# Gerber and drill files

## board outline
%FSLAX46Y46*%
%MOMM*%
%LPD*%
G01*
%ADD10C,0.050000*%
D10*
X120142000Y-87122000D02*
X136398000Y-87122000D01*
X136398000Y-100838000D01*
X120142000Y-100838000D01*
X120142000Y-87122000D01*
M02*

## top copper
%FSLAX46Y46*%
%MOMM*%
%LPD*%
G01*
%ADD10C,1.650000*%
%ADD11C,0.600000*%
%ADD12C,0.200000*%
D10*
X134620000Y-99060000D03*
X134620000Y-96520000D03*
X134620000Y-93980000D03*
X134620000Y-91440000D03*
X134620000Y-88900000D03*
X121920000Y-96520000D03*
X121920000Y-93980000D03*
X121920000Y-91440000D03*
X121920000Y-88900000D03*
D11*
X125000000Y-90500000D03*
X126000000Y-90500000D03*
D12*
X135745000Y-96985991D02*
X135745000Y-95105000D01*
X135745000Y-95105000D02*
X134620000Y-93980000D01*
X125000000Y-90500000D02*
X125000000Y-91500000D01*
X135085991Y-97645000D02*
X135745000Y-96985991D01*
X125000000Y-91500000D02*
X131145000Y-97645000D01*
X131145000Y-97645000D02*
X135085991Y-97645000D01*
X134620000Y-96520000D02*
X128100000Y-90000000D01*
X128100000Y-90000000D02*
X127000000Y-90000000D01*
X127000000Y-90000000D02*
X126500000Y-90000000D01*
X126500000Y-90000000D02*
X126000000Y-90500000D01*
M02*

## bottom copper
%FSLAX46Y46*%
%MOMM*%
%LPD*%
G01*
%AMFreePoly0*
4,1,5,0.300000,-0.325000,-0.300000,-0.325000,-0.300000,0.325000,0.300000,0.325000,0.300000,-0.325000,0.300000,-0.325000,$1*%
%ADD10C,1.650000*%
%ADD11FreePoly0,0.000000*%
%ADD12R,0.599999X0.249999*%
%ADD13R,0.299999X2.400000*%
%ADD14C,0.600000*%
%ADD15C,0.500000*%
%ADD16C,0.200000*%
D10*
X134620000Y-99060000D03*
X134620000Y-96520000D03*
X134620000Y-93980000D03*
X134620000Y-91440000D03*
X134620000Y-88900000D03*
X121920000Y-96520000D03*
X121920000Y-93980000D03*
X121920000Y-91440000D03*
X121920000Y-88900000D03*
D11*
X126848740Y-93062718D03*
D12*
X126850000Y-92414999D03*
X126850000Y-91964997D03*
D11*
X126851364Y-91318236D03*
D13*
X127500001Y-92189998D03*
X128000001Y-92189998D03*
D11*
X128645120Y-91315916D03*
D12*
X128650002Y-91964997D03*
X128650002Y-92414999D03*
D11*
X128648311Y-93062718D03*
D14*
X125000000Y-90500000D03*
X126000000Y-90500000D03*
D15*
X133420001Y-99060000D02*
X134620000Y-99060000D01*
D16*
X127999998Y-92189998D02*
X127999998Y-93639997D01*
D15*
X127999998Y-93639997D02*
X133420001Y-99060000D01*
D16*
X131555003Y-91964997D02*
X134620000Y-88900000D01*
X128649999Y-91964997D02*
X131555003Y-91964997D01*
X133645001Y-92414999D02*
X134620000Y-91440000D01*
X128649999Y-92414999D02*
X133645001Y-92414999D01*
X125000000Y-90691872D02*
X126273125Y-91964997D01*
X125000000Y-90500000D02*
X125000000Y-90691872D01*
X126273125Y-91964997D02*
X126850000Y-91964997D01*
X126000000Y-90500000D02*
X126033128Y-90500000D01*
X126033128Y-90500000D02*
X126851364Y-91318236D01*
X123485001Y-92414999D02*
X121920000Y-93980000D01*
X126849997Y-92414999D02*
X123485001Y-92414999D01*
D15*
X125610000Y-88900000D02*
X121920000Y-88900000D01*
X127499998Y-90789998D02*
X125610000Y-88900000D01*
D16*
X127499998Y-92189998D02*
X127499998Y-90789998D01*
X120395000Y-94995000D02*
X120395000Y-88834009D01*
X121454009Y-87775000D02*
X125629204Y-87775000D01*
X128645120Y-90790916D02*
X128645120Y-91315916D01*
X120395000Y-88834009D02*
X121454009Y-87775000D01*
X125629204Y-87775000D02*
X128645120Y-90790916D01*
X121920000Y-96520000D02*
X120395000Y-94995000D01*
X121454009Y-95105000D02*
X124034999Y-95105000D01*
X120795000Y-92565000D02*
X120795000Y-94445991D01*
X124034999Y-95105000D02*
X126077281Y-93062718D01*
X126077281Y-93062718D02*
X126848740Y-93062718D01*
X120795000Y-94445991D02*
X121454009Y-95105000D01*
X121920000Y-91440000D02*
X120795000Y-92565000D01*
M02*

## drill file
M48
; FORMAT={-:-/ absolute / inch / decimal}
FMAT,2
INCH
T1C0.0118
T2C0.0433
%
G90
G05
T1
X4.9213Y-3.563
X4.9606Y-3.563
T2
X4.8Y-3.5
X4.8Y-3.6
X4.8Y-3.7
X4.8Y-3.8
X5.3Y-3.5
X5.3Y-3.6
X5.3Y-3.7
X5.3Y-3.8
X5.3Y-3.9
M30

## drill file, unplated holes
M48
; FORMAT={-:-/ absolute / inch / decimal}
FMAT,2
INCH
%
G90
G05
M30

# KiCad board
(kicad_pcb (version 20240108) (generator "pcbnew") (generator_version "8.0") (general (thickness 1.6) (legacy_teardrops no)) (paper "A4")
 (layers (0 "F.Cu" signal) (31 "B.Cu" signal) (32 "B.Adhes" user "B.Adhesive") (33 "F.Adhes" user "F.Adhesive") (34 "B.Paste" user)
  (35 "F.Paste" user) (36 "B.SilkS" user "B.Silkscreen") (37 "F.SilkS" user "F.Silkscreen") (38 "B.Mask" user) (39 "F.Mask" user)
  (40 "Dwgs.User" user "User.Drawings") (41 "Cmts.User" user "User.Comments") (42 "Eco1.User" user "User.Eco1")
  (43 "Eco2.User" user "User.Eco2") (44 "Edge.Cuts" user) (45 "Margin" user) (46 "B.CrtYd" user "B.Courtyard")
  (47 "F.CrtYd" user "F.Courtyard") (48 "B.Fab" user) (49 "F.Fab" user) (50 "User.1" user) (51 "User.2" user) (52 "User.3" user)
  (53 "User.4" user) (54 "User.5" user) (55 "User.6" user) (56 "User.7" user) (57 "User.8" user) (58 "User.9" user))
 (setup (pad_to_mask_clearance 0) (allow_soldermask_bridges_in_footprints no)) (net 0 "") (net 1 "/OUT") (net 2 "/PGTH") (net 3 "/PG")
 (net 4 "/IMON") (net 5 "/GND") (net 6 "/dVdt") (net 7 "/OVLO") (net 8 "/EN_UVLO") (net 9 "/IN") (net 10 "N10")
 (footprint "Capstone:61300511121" (layer "F.Cu") (at 134.62 93.98 90)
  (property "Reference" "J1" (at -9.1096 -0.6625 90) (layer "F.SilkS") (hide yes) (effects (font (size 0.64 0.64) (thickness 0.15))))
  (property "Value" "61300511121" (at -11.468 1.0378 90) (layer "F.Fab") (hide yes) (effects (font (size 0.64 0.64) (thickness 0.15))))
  (pad "1" thru_hole circle (at -5.08 0 90) (size 1.65 1.65) (drill 1.1) (layers "*.Cu" "*.Mask") (remove_unused_layers no) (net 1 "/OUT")
   (solder_mask_margin 0.102))
  (pad "2" thru_hole circle (at -2.54 0 90) (size 1.65 1.65) (drill 1.1) (layers "*.Cu" "*.Mask") (remove_unused_layers no) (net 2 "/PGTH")
   (solder_mask_margin 0.102))
  (pad "3" thru_hole circle (at 0 0 90) (size 1.65 1.65) (drill 1.1) (layers "*.Cu" "*.Mask") (remove_unused_layers no) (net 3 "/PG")
   (solder_mask_margin 0.102))
  (pad "4" thru_hole circle (at 2.54 0 90) (size 1.65 1.65) (drill 1.1) (layers "*.Cu" "*.Mask") (remove_unused_layers no) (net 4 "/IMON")
   (solder_mask_margin 0.102))
  (pad "5" thru_hole circle (at 5.08 0 90) (size 1.65 1.65) (drill 1.1) (layers "*.Cu" "*.Mask") (remove_unused_layers no) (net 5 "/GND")
   (solder_mask_margin 0.102)))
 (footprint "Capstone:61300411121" (layer "F.Cu") (at 121.92 92.71 90)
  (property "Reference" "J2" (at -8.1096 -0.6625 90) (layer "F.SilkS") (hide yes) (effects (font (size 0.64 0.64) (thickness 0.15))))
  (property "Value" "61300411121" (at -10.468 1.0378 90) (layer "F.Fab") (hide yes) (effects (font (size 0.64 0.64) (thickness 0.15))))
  (pad "1" thru_hole circle (at -3.81 0 90) (size 1.65 1.65) (drill 1.1) (layers "*.Cu" "*.Mask") (remove_unused_layers no) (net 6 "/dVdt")
   (solder_mask_margin 0.102))
  (pad "2" thru_hole circle (at -1.27 0 90) (size 1.65 1.65) (drill 1.1) (layers "*.Cu" "*.Mask") (remove_unused_layers no) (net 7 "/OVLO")
   (solder_mask_margin 0.102))
  (pad "3" thru_hole circle (at 1.27 0 90) (size 1.65 1.65) (drill 1.1) (layers "*.Cu" "*.Mask") (remove_unused_layers no)
   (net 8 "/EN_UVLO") (solder_mask_margin 0.102))
  (pad "4" thru_hole circle (at 3.81 0 90) (size 1.65 1.65) (drill 1.1) (layers "*.Cu" "*.Mask") (remove_unused_layers no) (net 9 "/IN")
   (solder_mask_margin 0.102)))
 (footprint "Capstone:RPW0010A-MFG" (layer "B.Cu") (at 127.750001 92.189998)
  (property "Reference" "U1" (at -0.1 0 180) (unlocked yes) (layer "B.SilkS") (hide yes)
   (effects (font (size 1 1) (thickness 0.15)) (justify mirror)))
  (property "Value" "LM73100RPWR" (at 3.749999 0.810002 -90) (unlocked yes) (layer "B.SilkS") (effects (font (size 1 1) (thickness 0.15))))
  (pad "1" smd custom (at -0.901261 0.87272) (size 0.6 0.65) (layers "B.Cu" "B.Mask") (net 8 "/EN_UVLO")
   (options (clearance outline) (anchor rect)) (primitives))
  (pad "2" smd rect (at -0.900001 0.225001) (size 0.599999 0.249999) (layers "B.Cu" "B.Paste" "B.Mask") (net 7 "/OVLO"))
  (pad "3" smd rect (at -0.900001 -0.225001) (size 0.599999 0.249999) (layers "B.Cu" "B.Paste" "B.Mask") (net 3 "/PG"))
  (pad "4" smd custom (at -0.898637 -0.871762) (size 0.6 0.65) (layers "B.Cu" "B.Mask") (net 2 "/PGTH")
   (options (clearance outline) (anchor rect)) (primitives))
  (pad "5" smd rect (at -0.25 0) (size 0.299999 2.4) (layers "B.Cu" "B.Mask") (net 9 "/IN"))
  (pad "6" smd rect (at 0.25 0) (size 0.299999 2.4) (layers "B.Cu" "B.Mask") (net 1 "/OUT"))
  (pad "7" smd custom (at 0.895119 -0.874082) (size 0.6 0.65) (layers "B.Cu" "B.Mask") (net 6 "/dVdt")
   (options (clearance outline) (anchor rect)) (primitives))
  (pad "8" smd rect (at 0.900001 -0.225001) (size 0.599999 0.249999) (layers "B.Cu" "B.Paste" "B.Mask") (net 5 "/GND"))
  (pad "9" smd rect (at 0.900001 0.225001) (size 0.599999 0.249999) (layers "B.Cu" "B.Paste" "B.Mask") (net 4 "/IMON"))
  (pad "10" smd custom (at 0.89831 0.87272) (size 0.6 0.65) (layers "B.Cu" "B.Mask") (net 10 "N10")
   (options (clearance outline) (anchor rect)) (primitives)))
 (gr_rect (start 120.142 87.122) (end 136.398 100.838) (stroke (width 0.05) (type default)) (fill none) (layer "Edge.Cuts"))
 (segment (start 133.420001 99.06) (end 134.62 99.06) (width 0.5) (layer "B.Cu") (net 1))
 (segment (start 127.999998 92.189998) (end 127.999998 93.639997) (width 0.2) (layer "B.Cu") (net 1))
 (segment (start 127.999998 93.639997) (end 133.420001 99.06) (width 0.5) (layer "B.Cu") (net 1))
 (segment (start 131.555003 91.964997) (end 134.62 88.9) (width 0.2) (layer "B.Cu") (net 5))
 (segment (start 128.649999 91.964997) (end 131.555003 91.964997) (width 0.2) (layer "B.Cu") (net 5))
 (segment (start 133.645001 92.414999) (end 134.62 91.44) (width 0.2) (layer "B.Cu") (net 4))
 (segment (start 128.649999 92.414999) (end 133.645001 92.414999) (width 0.2) (layer "B.Cu") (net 4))
 (segment (start 135.745 96.985991) (end 135.745 95.105) (width 0.2) (layer "F.Cu") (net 3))
 (segment (start 135.745 95.105) (end 134.62 93.98) (width 0.2) (layer "F.Cu") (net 3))
 (segment (start 125 90.5) (end 125 91.5) (width 0.2) (layer "F.Cu") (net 3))
 (segment (start 135.085991 97.645) (end 135.745 96.985991) (width 0.2) (layer "F.Cu") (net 3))
 (segment (start 125 91.5) (end 131.145 97.645) (width 0.2) (layer "F.Cu") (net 3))
 (segment (start 131.145 97.645) (end 135.085991 97.645) (width 0.2) (layer "F.Cu") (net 3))
 (via (at 125 90.5) (size 0.6) (drill 0.3) (layers "F.Cu" "B.Cu") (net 3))
 (segment (start 125 90.691872) (end 126.273125 91.964997) (width 0.2) (layer "B.Cu") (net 3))
 (segment (start 125 90.5) (end 125 90.691872) (width 0.2) (layer "B.Cu") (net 3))
 (segment (start 126.273125 91.964997) (end 126.85 91.964997) (width 0.2) (layer "B.Cu") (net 3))
 (segment (start 134.62 96.52) (end 128.1 90) (width 0.2) (layer "F.Cu") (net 2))
 (segment (start 128.1 90) (end 127 90) (width 0.2) (layer "F.Cu") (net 2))
 (segment (start 127 90) (end 126.5 90) (width 0.2) (layer "F.Cu") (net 2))
 (segment (start 126.5 90) (end 126 90.5) (width 0.2) (layer "F.Cu") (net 2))
 (via (at 126 90.5) (size 0.6) (drill 0.3) (layers "F.Cu" "B.Cu") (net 2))
 (segment (start 126 90.5) (end 126.033128 90.5) (width 0.2) (layer "B.Cu") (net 2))
 (segment (start 126.033128 90.5) (end 126.851364 91.318236) (width 0.2) (layer "B.Cu") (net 2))
 (segment (start 123.485001 92.414999) (end 121.92 93.98) (width 0.2) (layer "B.Cu") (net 7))
 (segment (start 126.849997 92.414999) (end 123.485001 92.414999) (width 0.2) (layer "B.Cu") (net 7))
 (segment (start 125.61 88.9) (end 121.92 88.9) (width 0.5) (layer "B.Cu") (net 9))
 (segment (start 127.499998 90.789998) (end 125.61 88.9) (width 0.5) (layer "B.Cu") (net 9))
 (segment (start 127.499998 92.189998) (end 127.499998 90.789998) (width 0.2) (layer "B.Cu") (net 9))
 (segment (start 120.395 94.995) (end 120.395 88.834009) (width 0.2) (layer "B.Cu") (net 6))
 (segment (start 121.454009 87.775) (end 125.629204 87.775) (width 0.2) (layer "B.Cu") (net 6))
 (segment (start 128.64512 90.790916) (end 128.64512 91.315916) (width 0.2) (layer "B.Cu") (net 6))
 (segment (start 120.395 88.834009) (end 121.454009 87.775) (width 0.2) (layer "B.Cu") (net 6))
 (segment (start 125.629204 87.775) (end 128.64512 90.790916) (width 0.2) (layer "B.Cu") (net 6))
 (segment (start 121.92 96.52) (end 120.395 94.995) (width 0.2) (layer "B.Cu") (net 6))
 (segment (start 121.454009 95.105) (end 124.034999 95.105) (width 0.2) (layer "B.Cu") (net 8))
 (segment (start 120.795 92.565) (end 120.795 94.445991) (width 0.2) (layer "B.Cu") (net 8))
 (segment (start 124.034999 95.105) (end 126.077281 93.062718) (width 0.2) (layer "B.Cu") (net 8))
 (segment (start 126.077281 93.062718) (end 126.84874 93.062718) (width 0.2) (layer "B.Cu") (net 8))
 (segment (start 120.795 94.445991) (end 121.454009 95.105) (width 0.2) (layer "B.Cu") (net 8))
 (segment (start 121.92 91.44) (end 120.795 92.565) (width 0.2) (layer "B.Cu") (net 8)))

